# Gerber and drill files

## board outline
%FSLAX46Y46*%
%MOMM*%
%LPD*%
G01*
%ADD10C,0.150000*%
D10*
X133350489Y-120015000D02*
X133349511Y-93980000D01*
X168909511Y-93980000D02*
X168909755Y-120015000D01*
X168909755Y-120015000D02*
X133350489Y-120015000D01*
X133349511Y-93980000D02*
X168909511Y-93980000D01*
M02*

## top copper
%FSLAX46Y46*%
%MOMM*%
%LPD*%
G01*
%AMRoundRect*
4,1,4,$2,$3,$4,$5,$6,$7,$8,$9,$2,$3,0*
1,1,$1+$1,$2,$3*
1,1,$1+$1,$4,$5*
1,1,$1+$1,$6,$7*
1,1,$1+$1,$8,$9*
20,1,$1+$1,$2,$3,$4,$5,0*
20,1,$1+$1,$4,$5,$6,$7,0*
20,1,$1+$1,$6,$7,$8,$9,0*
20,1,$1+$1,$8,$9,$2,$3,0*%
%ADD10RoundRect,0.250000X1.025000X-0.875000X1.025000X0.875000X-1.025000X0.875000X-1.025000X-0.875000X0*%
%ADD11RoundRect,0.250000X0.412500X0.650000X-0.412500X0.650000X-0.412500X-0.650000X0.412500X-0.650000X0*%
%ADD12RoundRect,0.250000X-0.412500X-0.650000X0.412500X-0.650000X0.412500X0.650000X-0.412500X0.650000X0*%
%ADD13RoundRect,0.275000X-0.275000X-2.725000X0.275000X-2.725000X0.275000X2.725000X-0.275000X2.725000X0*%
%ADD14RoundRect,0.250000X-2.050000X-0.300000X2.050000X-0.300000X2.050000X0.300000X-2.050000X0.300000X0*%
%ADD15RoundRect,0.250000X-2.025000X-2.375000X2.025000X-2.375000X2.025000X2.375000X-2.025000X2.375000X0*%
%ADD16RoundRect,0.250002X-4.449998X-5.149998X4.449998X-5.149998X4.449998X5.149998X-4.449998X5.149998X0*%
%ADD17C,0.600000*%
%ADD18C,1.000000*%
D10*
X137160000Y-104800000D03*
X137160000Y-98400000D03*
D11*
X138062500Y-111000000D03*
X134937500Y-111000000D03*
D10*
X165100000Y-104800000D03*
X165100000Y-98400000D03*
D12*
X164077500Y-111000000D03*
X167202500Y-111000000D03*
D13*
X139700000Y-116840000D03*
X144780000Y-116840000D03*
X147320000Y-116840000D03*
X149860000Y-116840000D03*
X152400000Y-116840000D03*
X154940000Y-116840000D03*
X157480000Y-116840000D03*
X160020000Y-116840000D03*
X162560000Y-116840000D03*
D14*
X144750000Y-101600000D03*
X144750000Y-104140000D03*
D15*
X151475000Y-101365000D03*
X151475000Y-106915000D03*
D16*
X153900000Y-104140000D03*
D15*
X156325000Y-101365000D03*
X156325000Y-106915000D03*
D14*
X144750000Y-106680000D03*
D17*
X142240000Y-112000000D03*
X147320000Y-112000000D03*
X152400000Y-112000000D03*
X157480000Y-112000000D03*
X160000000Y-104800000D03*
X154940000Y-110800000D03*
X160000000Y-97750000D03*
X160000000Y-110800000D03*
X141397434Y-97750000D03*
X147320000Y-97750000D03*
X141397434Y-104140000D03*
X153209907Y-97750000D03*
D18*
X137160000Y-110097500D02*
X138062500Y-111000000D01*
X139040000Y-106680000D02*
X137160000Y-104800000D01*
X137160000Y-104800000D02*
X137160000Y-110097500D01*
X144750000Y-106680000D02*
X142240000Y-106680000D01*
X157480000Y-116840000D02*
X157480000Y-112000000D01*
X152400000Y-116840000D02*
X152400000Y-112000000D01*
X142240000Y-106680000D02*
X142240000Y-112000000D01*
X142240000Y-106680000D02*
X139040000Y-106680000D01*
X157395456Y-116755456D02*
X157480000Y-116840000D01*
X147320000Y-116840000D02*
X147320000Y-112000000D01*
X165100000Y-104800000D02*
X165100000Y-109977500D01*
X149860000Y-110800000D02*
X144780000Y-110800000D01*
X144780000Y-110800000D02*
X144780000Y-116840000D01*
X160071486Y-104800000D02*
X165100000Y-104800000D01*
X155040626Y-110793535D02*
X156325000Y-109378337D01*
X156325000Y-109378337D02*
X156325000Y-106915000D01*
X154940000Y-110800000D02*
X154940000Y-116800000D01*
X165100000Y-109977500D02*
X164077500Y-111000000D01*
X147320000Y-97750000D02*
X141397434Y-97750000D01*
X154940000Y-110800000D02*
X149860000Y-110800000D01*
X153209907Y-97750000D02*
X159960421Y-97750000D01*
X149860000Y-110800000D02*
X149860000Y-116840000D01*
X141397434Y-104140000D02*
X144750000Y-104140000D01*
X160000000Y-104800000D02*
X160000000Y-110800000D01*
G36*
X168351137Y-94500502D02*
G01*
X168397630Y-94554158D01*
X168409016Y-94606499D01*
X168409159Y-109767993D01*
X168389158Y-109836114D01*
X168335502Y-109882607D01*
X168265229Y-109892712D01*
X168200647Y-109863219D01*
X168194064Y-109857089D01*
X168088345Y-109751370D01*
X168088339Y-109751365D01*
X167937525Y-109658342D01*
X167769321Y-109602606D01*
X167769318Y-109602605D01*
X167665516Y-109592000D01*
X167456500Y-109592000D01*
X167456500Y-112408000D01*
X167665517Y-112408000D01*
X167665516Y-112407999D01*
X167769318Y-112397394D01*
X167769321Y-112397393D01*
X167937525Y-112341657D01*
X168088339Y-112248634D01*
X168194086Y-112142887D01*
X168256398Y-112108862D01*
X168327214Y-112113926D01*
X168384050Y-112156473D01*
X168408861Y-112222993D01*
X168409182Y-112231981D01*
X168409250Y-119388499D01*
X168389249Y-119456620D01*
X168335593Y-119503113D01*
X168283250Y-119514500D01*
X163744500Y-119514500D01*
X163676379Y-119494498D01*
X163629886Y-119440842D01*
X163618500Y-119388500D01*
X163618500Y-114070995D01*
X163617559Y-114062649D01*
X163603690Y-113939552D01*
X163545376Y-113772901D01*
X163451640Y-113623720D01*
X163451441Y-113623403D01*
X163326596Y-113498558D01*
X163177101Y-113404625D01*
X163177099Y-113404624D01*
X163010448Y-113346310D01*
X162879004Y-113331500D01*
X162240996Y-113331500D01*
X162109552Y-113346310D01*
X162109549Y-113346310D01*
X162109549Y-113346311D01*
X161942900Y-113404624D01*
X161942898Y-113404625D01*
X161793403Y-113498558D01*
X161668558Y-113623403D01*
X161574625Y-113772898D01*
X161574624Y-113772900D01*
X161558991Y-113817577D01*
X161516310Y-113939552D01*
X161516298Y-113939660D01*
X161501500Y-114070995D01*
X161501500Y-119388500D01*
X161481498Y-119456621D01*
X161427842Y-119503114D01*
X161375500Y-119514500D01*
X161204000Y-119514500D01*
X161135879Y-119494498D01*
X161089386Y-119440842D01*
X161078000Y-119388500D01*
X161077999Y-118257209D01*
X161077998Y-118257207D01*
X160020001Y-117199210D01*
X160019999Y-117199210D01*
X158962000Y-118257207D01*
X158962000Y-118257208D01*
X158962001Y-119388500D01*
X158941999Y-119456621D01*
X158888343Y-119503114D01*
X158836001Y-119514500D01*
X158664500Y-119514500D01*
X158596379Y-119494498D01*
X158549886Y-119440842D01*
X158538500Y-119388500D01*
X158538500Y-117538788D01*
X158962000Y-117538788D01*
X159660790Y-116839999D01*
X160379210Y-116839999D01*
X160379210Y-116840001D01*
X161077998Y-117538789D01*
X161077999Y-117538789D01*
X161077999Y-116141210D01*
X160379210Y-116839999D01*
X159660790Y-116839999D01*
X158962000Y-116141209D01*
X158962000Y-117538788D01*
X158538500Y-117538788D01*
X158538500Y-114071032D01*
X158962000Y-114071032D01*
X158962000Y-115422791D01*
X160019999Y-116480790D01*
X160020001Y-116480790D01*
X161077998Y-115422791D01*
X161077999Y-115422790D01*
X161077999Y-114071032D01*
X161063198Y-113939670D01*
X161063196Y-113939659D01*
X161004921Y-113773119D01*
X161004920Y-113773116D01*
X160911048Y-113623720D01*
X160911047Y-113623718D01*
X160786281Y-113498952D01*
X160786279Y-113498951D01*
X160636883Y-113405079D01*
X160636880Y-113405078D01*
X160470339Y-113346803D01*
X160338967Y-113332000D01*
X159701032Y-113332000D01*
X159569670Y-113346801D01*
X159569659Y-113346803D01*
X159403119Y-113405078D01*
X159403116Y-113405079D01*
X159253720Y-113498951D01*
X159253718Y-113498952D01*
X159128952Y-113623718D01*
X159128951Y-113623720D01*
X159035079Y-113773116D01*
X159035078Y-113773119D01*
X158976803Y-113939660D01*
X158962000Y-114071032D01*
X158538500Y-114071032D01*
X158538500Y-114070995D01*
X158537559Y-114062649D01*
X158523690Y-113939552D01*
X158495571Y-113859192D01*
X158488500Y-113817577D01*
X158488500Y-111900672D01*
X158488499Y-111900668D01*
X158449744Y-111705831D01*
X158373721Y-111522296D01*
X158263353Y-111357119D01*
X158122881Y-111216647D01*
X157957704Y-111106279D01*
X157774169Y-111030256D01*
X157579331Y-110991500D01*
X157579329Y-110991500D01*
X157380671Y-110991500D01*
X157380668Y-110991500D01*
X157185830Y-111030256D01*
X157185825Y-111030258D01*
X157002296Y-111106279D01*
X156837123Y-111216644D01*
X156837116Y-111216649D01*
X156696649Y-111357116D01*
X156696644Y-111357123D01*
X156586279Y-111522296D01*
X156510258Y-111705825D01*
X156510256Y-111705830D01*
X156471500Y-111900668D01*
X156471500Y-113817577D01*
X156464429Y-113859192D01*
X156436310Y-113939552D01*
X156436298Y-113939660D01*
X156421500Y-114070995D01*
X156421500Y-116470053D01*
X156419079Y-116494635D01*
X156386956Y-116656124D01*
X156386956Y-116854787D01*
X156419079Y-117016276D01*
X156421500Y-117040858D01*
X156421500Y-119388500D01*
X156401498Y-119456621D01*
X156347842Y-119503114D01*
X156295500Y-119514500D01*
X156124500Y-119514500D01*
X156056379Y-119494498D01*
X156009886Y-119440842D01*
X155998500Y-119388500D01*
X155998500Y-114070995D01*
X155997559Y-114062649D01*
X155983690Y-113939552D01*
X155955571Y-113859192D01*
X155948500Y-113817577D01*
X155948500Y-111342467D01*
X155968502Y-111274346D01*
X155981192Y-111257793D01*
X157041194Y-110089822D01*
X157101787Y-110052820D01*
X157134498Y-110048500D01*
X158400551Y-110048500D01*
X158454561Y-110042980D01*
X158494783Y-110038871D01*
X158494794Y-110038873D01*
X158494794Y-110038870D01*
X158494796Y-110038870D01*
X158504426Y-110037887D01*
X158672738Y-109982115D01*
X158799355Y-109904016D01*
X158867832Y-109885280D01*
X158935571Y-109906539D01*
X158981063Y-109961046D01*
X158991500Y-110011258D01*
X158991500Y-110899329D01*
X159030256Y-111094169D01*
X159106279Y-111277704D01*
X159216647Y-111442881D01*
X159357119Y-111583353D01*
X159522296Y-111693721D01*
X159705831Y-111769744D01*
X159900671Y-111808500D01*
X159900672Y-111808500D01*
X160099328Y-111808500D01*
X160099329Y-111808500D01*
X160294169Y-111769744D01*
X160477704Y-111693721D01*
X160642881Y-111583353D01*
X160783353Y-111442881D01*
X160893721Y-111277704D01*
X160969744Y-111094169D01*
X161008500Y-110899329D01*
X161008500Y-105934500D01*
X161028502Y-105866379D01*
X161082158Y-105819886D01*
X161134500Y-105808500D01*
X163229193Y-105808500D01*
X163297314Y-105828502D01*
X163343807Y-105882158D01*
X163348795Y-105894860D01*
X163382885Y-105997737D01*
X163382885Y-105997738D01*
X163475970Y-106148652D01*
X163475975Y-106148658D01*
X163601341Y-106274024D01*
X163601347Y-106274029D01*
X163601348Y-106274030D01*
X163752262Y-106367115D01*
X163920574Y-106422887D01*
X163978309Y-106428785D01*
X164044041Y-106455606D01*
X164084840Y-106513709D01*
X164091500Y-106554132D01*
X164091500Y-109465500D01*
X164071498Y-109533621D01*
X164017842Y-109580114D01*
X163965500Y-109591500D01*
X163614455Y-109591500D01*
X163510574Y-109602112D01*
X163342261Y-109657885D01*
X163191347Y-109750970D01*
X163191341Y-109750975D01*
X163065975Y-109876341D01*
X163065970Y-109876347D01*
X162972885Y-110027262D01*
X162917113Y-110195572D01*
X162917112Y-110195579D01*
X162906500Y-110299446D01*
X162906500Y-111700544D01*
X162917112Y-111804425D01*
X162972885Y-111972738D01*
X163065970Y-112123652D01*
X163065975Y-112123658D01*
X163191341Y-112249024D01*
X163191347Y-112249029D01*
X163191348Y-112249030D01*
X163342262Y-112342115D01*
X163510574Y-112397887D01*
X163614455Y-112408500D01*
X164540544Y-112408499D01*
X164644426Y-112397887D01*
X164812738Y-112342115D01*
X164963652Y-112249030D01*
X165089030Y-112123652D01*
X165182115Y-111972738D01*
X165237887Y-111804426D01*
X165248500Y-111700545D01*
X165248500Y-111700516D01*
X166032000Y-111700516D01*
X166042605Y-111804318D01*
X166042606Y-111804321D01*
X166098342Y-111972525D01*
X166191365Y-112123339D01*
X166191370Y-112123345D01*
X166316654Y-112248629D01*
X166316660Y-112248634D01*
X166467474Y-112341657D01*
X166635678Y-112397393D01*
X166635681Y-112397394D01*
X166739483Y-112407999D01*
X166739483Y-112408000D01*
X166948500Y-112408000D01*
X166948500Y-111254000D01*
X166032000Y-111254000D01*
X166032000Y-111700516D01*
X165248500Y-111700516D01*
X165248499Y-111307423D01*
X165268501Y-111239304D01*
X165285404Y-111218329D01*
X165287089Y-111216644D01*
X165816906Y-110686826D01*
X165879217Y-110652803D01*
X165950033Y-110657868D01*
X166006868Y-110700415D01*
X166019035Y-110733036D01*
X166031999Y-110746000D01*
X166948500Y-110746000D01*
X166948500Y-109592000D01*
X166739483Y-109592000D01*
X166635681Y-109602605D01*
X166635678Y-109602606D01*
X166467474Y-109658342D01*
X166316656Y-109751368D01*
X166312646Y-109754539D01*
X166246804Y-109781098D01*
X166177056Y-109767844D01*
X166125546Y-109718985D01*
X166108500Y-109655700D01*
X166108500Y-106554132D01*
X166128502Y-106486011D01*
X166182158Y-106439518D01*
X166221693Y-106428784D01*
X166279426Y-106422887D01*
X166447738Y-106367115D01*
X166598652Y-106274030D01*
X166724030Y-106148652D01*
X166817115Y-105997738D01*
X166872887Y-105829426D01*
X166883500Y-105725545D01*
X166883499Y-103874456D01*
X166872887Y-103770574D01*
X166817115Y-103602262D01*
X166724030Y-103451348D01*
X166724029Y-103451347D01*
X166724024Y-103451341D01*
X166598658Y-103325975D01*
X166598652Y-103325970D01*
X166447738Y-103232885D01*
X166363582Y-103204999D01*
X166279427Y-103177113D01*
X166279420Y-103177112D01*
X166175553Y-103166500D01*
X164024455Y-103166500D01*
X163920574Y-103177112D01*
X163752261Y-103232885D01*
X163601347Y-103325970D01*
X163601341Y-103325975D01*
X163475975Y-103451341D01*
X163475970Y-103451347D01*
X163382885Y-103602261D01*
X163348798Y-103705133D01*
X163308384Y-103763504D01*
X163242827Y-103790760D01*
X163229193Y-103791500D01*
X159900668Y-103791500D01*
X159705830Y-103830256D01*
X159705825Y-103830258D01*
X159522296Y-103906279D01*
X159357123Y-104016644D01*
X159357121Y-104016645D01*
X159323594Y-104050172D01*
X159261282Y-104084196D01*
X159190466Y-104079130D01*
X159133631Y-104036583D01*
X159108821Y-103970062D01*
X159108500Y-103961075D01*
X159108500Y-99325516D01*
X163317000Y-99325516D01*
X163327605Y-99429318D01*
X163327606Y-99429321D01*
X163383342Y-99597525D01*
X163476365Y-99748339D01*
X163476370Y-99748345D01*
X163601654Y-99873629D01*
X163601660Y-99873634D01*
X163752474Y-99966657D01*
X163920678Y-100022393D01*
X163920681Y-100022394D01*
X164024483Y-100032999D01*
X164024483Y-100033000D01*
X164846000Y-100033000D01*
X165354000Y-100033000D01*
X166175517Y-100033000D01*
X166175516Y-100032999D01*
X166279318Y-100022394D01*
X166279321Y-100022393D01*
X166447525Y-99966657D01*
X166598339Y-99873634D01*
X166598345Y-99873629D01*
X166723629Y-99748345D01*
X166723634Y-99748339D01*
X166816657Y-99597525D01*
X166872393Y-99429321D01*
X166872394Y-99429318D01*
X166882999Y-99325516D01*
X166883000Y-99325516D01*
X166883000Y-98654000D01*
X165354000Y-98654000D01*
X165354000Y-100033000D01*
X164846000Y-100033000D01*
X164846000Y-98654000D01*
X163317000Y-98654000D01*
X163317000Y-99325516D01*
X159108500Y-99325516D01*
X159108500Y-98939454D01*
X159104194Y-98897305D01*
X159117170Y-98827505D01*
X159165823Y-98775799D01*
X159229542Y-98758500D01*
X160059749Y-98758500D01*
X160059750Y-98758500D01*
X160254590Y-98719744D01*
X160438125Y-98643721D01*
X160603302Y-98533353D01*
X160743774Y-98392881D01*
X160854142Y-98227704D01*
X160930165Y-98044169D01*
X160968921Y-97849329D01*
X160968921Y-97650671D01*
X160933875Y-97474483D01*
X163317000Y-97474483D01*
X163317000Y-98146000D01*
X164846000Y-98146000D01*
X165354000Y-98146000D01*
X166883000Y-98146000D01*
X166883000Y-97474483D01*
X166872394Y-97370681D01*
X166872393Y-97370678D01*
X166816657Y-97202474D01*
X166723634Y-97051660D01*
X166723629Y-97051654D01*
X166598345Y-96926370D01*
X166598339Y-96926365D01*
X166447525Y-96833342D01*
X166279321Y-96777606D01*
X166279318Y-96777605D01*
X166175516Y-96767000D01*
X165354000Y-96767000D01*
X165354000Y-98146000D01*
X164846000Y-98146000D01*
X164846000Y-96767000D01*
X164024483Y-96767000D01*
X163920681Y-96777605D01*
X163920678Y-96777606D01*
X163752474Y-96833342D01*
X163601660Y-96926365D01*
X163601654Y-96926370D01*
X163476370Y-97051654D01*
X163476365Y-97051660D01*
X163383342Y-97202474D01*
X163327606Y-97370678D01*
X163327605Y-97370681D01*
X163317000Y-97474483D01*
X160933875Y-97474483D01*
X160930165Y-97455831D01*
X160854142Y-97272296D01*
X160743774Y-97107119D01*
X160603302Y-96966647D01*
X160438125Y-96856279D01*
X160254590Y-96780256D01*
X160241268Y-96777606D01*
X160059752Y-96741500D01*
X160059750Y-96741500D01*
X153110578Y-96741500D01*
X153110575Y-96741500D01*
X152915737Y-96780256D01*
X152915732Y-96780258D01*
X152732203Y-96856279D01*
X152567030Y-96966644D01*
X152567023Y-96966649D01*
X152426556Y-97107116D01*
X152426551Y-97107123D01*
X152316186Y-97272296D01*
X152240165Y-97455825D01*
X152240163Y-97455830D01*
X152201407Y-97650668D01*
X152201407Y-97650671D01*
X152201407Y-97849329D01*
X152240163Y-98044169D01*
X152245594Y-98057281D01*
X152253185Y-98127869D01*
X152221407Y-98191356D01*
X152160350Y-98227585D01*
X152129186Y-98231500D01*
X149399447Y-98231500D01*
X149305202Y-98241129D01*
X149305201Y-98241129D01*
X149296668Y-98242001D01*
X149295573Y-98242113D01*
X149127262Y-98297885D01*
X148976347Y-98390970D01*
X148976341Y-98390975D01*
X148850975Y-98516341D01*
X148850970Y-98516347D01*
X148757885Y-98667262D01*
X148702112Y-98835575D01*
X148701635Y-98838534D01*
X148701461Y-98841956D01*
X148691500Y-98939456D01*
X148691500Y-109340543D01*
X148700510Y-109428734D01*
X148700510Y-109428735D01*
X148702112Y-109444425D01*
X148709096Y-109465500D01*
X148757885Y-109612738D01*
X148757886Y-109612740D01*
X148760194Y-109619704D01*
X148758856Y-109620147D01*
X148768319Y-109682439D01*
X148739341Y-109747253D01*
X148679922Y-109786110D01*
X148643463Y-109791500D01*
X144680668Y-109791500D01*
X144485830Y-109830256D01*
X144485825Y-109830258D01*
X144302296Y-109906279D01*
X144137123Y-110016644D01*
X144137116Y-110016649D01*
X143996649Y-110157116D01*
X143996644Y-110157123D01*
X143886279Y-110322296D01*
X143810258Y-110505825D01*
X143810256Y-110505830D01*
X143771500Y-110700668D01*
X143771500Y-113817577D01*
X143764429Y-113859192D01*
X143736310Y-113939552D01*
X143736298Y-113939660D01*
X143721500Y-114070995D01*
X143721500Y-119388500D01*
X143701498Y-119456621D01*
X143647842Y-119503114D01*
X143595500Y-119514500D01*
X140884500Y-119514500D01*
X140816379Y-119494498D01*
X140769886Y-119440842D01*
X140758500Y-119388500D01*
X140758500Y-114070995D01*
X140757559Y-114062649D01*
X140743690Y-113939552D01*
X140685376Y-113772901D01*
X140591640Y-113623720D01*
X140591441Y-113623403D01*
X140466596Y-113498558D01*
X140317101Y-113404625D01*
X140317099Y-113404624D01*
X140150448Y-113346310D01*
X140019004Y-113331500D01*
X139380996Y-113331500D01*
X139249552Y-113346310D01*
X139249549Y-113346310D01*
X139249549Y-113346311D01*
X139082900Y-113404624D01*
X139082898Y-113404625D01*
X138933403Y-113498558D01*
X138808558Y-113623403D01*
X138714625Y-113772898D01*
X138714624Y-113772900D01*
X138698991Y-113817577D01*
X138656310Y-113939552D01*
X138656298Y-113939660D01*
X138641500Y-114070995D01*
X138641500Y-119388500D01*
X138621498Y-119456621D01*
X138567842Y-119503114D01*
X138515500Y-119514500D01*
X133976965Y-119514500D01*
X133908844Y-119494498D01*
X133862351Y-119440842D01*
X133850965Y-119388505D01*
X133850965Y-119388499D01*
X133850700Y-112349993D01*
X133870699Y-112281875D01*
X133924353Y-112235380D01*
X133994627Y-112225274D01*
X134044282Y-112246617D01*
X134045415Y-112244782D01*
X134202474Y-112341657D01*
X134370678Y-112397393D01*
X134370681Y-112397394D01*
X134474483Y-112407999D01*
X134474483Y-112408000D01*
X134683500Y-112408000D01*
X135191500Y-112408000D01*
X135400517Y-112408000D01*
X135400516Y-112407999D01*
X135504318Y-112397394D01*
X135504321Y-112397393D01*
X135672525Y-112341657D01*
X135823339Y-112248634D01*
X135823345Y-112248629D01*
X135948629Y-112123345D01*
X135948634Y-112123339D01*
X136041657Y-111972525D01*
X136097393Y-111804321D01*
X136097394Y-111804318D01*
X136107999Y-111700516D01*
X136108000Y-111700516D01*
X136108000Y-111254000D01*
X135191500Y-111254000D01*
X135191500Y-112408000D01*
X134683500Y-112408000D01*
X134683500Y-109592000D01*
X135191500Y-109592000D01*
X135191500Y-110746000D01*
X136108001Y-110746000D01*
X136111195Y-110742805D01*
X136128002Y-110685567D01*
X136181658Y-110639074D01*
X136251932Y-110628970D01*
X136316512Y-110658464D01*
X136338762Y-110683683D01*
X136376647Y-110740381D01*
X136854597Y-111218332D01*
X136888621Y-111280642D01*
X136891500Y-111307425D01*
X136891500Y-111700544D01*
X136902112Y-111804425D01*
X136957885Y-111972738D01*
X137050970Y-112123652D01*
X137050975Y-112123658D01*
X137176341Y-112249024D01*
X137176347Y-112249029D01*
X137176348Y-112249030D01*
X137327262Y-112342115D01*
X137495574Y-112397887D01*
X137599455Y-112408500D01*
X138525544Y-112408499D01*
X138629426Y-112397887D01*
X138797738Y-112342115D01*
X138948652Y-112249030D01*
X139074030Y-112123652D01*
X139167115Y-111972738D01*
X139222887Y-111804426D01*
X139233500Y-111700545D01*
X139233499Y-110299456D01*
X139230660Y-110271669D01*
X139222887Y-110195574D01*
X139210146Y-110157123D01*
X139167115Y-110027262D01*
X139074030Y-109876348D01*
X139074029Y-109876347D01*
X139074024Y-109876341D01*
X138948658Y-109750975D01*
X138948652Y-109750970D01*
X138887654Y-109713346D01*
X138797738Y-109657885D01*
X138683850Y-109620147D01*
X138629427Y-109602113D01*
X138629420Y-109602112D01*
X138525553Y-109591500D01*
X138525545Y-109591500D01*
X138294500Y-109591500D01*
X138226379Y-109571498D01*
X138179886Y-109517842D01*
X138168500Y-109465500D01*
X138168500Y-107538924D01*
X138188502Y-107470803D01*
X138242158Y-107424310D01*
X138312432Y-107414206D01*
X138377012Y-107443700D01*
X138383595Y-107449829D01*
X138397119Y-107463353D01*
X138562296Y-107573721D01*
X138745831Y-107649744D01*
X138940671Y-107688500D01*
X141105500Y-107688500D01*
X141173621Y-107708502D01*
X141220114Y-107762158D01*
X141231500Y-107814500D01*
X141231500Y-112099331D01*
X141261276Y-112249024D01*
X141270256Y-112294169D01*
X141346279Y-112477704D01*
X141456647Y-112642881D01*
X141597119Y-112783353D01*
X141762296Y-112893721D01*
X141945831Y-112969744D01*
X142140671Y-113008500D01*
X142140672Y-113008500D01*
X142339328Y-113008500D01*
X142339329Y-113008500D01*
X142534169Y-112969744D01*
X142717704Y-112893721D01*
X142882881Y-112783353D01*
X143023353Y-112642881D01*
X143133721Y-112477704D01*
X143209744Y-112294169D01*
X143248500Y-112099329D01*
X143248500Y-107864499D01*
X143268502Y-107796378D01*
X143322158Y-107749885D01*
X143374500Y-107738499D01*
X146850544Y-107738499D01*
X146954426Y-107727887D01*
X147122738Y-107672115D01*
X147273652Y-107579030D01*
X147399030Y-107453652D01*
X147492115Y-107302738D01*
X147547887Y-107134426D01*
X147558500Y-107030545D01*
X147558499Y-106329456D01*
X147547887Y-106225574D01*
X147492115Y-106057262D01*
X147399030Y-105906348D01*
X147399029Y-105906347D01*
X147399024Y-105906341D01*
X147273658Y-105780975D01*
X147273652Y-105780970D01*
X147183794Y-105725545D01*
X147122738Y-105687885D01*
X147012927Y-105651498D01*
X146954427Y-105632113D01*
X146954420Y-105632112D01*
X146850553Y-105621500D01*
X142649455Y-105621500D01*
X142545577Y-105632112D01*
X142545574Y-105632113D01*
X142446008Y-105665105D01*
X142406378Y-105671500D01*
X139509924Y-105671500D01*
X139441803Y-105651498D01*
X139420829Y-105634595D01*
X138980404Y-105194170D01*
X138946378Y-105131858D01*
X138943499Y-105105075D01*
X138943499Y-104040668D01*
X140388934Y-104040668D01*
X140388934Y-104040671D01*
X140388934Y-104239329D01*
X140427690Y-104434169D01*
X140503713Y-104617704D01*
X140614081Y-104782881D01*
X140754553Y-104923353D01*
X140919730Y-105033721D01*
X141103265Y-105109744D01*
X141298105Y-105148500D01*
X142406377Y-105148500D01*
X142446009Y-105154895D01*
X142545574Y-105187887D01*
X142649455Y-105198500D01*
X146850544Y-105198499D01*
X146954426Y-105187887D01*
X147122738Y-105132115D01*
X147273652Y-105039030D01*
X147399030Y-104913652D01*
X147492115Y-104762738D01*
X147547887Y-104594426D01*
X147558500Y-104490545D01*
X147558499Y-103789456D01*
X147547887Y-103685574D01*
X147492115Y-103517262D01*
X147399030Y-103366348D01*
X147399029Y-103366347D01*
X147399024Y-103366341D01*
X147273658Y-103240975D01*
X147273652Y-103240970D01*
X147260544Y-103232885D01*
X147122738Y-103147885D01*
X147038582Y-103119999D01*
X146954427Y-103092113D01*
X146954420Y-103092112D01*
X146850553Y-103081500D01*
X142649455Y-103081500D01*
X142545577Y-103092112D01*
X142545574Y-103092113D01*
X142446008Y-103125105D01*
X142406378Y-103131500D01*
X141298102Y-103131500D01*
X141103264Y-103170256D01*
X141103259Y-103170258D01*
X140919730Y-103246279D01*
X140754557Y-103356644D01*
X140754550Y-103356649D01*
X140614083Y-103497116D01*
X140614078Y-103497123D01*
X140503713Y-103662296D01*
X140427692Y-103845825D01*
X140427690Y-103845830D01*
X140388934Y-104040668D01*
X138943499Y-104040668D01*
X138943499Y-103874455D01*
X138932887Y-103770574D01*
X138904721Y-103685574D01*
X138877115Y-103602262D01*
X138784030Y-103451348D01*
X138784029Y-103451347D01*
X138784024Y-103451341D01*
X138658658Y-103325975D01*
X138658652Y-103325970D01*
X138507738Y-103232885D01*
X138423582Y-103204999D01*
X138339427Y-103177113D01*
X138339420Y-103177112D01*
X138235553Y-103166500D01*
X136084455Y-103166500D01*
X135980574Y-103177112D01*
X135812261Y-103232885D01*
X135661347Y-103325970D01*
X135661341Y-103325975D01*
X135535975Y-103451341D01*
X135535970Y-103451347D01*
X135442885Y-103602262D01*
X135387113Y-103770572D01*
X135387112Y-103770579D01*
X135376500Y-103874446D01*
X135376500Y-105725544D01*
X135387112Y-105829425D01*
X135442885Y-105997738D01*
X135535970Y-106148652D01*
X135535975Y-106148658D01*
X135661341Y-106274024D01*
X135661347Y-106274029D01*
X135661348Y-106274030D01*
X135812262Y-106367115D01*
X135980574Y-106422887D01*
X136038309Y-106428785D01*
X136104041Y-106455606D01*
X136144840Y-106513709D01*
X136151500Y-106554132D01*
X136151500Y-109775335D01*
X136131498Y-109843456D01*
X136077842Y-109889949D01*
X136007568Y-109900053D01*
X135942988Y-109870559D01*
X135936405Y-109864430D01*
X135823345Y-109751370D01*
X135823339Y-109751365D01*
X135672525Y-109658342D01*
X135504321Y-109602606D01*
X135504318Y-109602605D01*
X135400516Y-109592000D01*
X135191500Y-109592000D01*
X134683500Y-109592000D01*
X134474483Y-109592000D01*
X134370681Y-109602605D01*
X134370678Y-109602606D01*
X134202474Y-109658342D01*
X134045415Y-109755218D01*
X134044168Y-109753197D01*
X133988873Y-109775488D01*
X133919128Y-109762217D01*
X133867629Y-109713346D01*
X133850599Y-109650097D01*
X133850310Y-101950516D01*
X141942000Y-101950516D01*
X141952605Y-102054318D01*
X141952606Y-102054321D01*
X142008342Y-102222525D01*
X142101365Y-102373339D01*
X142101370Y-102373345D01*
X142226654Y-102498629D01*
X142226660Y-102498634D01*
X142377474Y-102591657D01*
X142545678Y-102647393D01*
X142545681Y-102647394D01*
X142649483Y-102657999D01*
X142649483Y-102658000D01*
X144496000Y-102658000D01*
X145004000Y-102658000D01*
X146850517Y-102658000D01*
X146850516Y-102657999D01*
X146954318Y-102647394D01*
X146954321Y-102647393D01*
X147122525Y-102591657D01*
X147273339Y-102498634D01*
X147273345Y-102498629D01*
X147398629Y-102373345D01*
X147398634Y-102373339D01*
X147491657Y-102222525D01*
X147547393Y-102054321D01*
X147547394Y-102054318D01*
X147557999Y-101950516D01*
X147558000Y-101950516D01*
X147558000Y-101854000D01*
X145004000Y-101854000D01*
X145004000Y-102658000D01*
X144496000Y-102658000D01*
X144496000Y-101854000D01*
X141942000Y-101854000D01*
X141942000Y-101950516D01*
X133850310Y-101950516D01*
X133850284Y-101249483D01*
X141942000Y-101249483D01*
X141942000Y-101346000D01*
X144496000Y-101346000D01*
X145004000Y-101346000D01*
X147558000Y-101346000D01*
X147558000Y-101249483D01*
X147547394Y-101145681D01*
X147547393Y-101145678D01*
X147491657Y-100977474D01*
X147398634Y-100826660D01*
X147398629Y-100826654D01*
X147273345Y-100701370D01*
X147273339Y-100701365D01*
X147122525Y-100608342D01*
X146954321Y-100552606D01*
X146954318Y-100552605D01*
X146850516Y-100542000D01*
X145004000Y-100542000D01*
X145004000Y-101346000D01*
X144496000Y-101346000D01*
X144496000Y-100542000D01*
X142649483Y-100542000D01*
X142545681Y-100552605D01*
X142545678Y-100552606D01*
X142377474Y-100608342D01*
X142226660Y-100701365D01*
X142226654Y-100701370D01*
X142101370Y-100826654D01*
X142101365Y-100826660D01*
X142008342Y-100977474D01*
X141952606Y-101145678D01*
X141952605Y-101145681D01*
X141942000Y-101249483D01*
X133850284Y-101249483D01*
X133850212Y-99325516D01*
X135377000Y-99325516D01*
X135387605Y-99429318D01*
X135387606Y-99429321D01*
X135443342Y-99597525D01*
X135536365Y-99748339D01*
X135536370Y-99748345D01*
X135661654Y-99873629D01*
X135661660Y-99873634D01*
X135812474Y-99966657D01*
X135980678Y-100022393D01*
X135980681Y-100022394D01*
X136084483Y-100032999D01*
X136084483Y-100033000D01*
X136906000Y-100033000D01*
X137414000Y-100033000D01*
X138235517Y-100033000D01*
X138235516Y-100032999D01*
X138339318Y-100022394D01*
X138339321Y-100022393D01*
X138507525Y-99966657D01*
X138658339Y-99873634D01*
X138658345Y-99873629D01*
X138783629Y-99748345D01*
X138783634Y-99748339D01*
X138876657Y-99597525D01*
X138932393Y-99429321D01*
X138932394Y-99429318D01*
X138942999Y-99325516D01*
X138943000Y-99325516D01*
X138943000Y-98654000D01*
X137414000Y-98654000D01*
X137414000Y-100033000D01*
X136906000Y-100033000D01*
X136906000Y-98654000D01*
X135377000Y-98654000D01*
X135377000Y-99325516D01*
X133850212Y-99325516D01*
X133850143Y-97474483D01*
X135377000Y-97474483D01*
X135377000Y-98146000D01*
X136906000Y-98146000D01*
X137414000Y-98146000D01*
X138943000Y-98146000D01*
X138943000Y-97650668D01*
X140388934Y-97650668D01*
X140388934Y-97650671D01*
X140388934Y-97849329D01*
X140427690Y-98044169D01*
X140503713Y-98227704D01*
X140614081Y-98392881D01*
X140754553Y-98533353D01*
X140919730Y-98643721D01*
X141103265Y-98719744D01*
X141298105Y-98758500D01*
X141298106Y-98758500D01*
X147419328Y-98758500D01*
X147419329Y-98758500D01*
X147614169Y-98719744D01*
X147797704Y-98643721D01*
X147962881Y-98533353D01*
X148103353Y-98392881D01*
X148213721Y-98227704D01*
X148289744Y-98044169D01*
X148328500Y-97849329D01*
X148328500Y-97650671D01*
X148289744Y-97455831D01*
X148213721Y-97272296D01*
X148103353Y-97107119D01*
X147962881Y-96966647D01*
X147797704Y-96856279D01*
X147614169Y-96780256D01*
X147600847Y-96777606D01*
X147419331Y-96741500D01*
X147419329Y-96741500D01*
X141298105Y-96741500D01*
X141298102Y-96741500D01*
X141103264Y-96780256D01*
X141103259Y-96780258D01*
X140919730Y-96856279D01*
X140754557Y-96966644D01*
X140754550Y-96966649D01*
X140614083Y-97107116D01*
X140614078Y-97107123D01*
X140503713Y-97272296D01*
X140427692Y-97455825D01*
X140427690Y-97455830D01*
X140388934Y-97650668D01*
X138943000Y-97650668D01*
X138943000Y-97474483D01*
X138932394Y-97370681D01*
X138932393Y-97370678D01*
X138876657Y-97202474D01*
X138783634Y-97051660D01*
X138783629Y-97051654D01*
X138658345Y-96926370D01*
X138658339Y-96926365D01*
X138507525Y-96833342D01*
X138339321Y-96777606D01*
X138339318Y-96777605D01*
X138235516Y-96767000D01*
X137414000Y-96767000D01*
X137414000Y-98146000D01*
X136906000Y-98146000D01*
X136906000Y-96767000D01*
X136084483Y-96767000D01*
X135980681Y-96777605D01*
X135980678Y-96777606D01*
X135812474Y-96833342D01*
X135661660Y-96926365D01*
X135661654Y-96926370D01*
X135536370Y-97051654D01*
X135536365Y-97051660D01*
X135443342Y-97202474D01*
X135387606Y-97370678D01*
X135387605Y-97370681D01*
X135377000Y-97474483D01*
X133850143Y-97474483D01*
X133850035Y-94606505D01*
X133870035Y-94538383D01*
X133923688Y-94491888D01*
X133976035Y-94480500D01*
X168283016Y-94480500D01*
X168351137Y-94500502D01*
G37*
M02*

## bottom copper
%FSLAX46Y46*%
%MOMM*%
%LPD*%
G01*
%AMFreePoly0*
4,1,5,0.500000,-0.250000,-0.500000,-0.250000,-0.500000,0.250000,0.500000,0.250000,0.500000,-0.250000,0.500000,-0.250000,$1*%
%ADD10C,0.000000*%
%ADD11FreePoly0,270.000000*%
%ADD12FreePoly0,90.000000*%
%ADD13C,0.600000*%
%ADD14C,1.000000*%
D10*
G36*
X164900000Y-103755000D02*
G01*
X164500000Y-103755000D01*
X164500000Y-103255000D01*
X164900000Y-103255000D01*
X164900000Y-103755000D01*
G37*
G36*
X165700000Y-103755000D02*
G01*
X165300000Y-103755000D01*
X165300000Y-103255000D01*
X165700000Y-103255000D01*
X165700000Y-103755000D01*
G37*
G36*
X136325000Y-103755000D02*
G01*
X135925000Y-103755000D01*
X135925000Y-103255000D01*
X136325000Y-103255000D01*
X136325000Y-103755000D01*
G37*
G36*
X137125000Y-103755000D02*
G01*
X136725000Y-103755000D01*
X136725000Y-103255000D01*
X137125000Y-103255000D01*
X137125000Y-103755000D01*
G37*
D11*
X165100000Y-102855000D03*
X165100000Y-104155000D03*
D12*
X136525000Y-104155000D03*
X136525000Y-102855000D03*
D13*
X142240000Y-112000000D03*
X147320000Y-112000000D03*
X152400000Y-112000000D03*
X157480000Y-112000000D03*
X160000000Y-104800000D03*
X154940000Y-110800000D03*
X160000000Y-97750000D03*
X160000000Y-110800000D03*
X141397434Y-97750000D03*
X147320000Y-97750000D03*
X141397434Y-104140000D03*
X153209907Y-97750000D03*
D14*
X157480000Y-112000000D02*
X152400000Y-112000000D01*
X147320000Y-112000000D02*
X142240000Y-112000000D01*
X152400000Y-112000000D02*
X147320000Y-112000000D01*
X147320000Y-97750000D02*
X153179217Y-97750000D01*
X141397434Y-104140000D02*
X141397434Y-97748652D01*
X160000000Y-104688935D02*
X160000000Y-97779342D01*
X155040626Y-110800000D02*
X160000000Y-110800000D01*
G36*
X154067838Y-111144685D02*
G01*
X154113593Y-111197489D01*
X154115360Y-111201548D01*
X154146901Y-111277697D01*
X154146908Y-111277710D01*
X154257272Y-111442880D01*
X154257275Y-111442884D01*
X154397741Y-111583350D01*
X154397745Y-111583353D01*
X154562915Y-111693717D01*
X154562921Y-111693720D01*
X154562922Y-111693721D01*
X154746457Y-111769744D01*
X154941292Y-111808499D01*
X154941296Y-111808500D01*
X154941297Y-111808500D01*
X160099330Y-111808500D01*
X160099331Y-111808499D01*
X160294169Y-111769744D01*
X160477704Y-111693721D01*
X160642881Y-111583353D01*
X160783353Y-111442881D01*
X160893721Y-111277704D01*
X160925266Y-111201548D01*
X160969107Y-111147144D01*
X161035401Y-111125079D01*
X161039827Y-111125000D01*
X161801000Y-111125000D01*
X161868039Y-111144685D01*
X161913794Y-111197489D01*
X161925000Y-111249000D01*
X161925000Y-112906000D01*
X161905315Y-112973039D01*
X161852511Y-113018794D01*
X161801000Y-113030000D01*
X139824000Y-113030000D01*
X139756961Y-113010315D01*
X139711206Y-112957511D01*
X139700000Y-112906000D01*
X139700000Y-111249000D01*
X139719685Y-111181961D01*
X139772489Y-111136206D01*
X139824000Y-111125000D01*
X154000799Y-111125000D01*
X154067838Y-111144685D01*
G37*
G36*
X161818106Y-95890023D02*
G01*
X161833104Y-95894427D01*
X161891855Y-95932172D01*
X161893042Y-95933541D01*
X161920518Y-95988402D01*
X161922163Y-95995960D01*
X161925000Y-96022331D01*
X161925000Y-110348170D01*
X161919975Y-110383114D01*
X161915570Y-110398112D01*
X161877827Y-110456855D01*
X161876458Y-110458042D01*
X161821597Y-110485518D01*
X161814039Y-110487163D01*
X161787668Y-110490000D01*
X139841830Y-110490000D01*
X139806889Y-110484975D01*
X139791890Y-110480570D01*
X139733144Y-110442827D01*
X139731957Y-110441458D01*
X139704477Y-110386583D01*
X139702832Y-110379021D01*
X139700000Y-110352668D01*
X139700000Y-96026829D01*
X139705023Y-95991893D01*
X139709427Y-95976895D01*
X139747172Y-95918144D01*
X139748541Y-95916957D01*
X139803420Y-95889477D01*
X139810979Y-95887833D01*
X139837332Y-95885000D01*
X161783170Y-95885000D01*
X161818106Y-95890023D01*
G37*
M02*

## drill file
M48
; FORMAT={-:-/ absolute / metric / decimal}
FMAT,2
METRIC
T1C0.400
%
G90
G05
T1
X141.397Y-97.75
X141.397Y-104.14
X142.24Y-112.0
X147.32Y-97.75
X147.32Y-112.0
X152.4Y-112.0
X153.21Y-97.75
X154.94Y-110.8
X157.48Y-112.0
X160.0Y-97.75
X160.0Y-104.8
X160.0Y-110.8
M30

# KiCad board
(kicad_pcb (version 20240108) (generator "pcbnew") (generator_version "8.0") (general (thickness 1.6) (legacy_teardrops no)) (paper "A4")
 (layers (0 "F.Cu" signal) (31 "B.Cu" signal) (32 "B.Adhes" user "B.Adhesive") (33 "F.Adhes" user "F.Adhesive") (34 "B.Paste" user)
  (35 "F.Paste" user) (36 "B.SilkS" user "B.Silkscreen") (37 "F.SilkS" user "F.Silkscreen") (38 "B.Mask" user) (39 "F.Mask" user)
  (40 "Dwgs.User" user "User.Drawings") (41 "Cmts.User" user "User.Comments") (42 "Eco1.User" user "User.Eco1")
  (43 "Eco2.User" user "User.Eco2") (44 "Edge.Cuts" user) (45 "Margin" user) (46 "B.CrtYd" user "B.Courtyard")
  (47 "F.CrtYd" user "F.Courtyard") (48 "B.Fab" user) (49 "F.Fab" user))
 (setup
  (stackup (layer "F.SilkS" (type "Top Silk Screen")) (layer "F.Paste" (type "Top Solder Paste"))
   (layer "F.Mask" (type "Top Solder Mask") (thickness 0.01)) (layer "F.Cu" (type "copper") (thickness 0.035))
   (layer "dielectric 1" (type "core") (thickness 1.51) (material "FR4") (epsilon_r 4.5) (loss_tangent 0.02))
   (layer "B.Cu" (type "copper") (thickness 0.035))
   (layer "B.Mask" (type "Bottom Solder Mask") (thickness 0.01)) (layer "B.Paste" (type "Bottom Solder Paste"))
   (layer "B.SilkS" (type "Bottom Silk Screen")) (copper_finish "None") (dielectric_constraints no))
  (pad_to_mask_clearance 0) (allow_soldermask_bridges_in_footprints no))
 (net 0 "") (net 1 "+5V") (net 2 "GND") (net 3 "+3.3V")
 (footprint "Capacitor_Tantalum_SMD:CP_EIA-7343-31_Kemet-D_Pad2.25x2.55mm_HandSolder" (layer "F.Cu") (at 137.16 101.6 90)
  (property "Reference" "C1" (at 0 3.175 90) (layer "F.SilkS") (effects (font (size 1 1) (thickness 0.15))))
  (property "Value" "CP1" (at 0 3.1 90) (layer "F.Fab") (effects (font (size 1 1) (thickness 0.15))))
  (pad "1" smd roundrect (at -3.2 0 90) (size 2.25 2.55) (layers "F.Cu" "F.Paste" "F.Mask") (roundrect_rratio 0.111111) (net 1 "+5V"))
  (pad "2" smd roundrect (at 3.2 0 90) (size 2.25 2.55) (layers "F.Cu" "F.Paste" "F.Mask") (roundrect_rratio 0.111111) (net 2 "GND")))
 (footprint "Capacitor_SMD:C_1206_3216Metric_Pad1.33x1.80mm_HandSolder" (layer "F.Cu") (at 136.5 111 180)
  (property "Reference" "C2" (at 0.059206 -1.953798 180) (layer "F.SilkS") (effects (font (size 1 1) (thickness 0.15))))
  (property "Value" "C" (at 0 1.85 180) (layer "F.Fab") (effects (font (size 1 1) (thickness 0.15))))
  (pad "1" smd roundrect (at -1.5625 0 180) (size 1.325 1.8) (layers "F.Cu" "F.Paste" "F.Mask") (roundrect_rratio 0.188679) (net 1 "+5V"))
  (pad "2" smd roundrect (at 1.5625 0 180) (size 1.325 1.8) (layers "F.Cu" "F.Paste" "F.Mask") (roundrect_rratio 0.188679) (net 2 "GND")))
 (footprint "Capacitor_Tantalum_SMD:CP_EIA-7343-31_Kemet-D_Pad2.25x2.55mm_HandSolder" (layer "F.Cu") (at 165.1 101.6 90)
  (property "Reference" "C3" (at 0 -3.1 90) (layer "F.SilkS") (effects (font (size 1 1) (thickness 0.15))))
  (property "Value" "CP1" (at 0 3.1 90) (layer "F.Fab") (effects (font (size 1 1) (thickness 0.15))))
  (pad "1" smd roundrect (at -3.2 0 90) (size 2.25 2.55) (layers "F.Cu" "F.Paste" "F.Mask") (roundrect_rratio 0.111111) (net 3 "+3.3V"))
  (pad "2" smd roundrect (at 3.2 0 90) (size 2.25 2.55) (layers "F.Cu" "F.Paste" "F.Mask") (roundrect_rratio 0.111111) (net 2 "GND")))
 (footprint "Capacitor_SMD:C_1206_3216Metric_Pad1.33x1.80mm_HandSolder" (layer "F.Cu") (at 165.64 111)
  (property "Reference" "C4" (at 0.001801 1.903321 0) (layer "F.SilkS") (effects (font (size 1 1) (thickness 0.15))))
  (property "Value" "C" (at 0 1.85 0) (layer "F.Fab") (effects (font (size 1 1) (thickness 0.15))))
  (pad "1" smd roundrect (at -1.5625 0) (size 1.325 1.8) (layers "F.Cu" "F.Paste" "F.Mask") (roundrect_rratio 0.188679) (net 3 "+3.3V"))
  (pad "2" smd roundrect (at 1.5625 0) (size 1.325 1.8) (layers "F.Cu" "F.Paste" "F.Mask") (roundrect_rratio 0.188679) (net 2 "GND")))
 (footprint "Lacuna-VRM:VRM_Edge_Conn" (layer "F.Cu") (at 157.48 124.46)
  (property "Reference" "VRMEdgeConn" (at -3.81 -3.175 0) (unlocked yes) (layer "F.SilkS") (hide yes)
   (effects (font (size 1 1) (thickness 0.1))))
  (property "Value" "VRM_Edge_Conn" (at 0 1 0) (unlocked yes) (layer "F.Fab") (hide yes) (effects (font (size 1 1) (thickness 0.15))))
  (pad "VC1" smd roundrect (at -17.78 -7.62) (size 1.1 6) (layers "F.Cu" "F.Paste" "F.Mask") (roundrect_rratio 0.25)
   (thermal_bridge_angle 45))
  (pad "VC2" smd roundrect (at -12.7 -7.62) (size 1.1 6) (layers "F.Cu" "F.Paste" "F.Mask") (roundrect_rratio 0.25) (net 3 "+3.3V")
   (thermal_bridge_angle 45))
  (pad "VC3" smd roundrect (at -10.16 -7.62) (size 1.1 6) (layers "F.Cu" "F.Paste" "F.Mask") (roundrect_rratio 0.25) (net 1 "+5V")
   (thermal_bridge_angle 45))
  (pad "VC4" smd roundrect (at -7.62 -7.62) (size 1.1 6) (layers "F.Cu" "F.Paste" "F.Mask") (roundrect_rratio 0.25) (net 3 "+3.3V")
   (thermal_bridge_angle 45))
  (pad "VC5" smd roundrect (at -5.08 -7.62) (size 1.1 6) (layers "F.Cu" "F.Paste" "F.Mask") (roundrect_rratio 0.25) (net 1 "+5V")
   (thermal_bridge_angle 45))
  (pad "VC6" smd roundrect (at -2.54 -7.62) (size 1.1 6) (layers "F.Cu" "F.Paste" "F.Mask") (roundrect_rratio 0.25) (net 3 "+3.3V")
   (thermal_bridge_angle 45))
  (pad "VC7" smd roundrect (at 0 -7.62) (size 1.1 6) (layers "F.Cu" "F.Paste" "F.Mask") (roundrect_rratio 0.25) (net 1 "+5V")
   (thermal_bridge_angle 45))
  (pad "VC8" smd roundrect (at 2.54 -7.62) (size 1.1 6) (layers "F.Cu" "F.Paste" "F.Mask") (roundrect_rratio 0.25) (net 2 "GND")
   (thermal_bridge_angle 45))
  (pad "VC9" smd roundrect (at 5.08 -7.62) (size 1.1 6) (layers "F.Cu" "F.Paste" "F.Mask") (roundrect_rratio 0.25) (thermal_bridge_angle 45)))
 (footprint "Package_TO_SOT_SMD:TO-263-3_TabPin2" (layer "F.Cu") (at 152.4 104.14)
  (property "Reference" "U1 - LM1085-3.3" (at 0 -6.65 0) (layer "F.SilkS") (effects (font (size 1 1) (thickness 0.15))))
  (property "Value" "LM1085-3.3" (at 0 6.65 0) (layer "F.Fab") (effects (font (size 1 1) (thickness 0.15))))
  (pad "1" smd roundrect (at -7.65 -2.54) (size 4.6 1.1) (layers "F.Cu" "F.Paste" "F.Mask") (roundrect_rratio 0.227273) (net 2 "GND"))
  (pad "2" smd roundrect (at -7.65 0) (size 4.6 1.1) (layers "F.Cu" "F.Paste" "F.Mask") (roundrect_rratio 0.227273) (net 3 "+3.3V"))
  (pad "2" smd roundrect (at -0.925 -2.775) (size 4.55 5.25) (layers "F.Cu" "F.Paste") (roundrect_rratio 0.054945) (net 3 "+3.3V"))
  (pad "2" smd roundrect (at -0.925 2.775) (size 4.55 5.25) (layers "F.Cu" "F.Paste") (roundrect_rratio 0.054945) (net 3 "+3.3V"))
  (pad "2" smd roundrect (at 1.5 0) (size 9.4 10.8) (layers "F.Cu" "F.Mask") (roundrect_rratio 0.026596) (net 3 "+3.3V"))
  (pad "2" smd roundrect (at 3.925 -2.775) (size 4.55 5.25) (layers "F.Cu" "F.Paste") (roundrect_rratio 0.054945) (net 3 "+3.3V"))
  (pad "2" smd roundrect (at 3.925 2.775) (size 4.55 5.25) (layers "F.Cu" "F.Paste") (roundrect_rratio 0.054945) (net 3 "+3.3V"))
  (pad "3" smd roundrect (at -7.65 2.54) (size 4.6 1.1) (layers "F.Cu" "F.Paste" "F.Mask") (roundrect_rratio 0.227273) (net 1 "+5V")))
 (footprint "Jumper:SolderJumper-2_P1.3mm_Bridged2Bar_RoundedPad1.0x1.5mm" (layer "B.Cu") (at 165.1 103.505 -90)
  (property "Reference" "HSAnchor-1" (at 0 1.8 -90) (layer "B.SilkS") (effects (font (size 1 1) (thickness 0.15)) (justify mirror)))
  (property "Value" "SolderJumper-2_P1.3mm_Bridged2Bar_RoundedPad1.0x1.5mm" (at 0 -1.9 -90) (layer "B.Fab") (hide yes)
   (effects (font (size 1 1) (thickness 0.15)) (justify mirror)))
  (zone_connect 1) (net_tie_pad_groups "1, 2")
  (fp_poly (pts (xy -0.25 0.6) (xy 0.25 0.6) (xy 0.25 0.2) (xy -0.25 0.2)) (stroke (width 0) (type solid)) (fill solid) (layer "B.Cu"))
  (fp_poly (pts (xy -0.25 -0.2) (xy 0.25 -0.2) (xy 0.25 -0.6) (xy -0.25 -0.6)) (stroke (width 0) (type solid)) (fill solid) (layer "B.Cu"))
  (pad "1" smd custom (at -0.65 0 270) (size 1 0.5) (layers "B.Cu" "B.Mask") (zone_connect 2) (thermal_bridge_angle 45)
   (options (clearance outline) (anchor rect)) (primitives))
  (pad "2" smd custom (at 0.65 0 270) (size 1 0.5) (layers "B.Cu" "B.Mask") (zone_connect 2) (thermal_bridge_angle 45)
   (options (clearance outline) (anchor rect)) (primitives)))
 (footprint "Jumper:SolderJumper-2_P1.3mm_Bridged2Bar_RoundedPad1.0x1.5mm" (layer "B.Cu") (at 136.525 103.505 90)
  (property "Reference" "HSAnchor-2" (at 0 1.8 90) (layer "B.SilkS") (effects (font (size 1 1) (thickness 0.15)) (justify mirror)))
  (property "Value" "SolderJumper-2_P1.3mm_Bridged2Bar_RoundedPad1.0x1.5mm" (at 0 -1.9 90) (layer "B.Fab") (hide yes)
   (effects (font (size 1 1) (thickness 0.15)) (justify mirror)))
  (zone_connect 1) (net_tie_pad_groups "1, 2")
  (fp_poly (pts (xy -0.25 -0.2) (xy 0.25 -0.2) (xy 0.25 -0.6) (xy -0.25 -0.6)) (stroke (width 0) (type solid)) (fill solid) (layer "B.Cu"))
  (fp_poly (pts (xy -0.25 0.6) (xy 0.25 0.6) (xy 0.25 0.2) (xy -0.25 0.2)) (stroke (width 0) (type solid)) (fill solid) (layer "B.Cu"))
  (pad "1" smd custom (at -0.65 0 90) (size 1 0.5) (layers "B.Cu" "B.Mask") (zone_connect 2) (thermal_bridge_angle 45)
   (options (clearance outline) (anchor rect)) (primitives))
  (pad "2" smd custom (at 0.65 0 90) (size 1 0.5) (layers "B.Cu" "B.Mask") (zone_connect 2) (thermal_bridge_angle 45)
   (options (clearance outline) (anchor rect)) (primitives)))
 (gr_line (start 133.350489 120.015) (end 133.349511 93.98) (stroke (width 0.15) (type default)) (layer "Edge.Cuts"))
 (gr_line (start 168.909511 93.98) (end 168.909755 120.015) (stroke (width 0.15) (type default)) (layer "Edge.Cuts"))
 (gr_line (start 168.909755 120.015) (end 133.350489 120.015) (stroke (width 0.15) (type default)) (layer "Edge.Cuts"))
 (gr_line (start 133.349511 93.98) (end 168.909511 93.98) (stroke (width 0.15) (type default)) (layer "Edge.Cuts"))
 (segment (start 137.16 110.0975) (end 138.0625 111) (width 1) (layer "F.Cu") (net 1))
 (segment (start 139.04 106.68) (end 137.16 104.8) (width 1) (layer "F.Cu") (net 1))
 (segment (start 137.16 104.8) (end 137.16 110.0975) (width 1) (layer "F.Cu") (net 1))
 (segment (start 144.75 106.68) (end 142.24 106.68) (width 1) (layer "F.Cu") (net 1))
 (segment (start 157.48 116.84) (end 157.48 112) (width 1) (layer "F.Cu") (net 1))
 (segment (start 152.4 116.84) (end 152.4 112) (width 1) (layer "F.Cu") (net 1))
 (segment (start 142.24 106.68) (end 142.24 112) (width 1) (layer "F.Cu") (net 1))
 (segment (start 142.24 106.68) (end 139.04 106.68) (width 1) (layer "F.Cu") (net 1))
 (segment (start 157.395456 116.755456) (end 157.48 116.84) (width 1) (layer "F.Cu") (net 1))
 (segment (start 147.32 116.84) (end 147.32 112) (width 1) (layer "F.Cu") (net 1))
 (via (at 142.24 112) (size 0.6) (drill 0.4) (layers "F.Cu" "B.Cu") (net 1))
 (via (at 147.32 112) (size 0.6) (drill 0.4) (layers "F.Cu" "B.Cu") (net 1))
 (via (at 152.4 112) (size 0.6) (drill 0.4) (layers "F.Cu" "B.Cu") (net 1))
 (via (at 157.48 112) (size 0.6) (drill 0.4) (layers "F.Cu" "B.Cu") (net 1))
 (segment (start 157.48 112) (end 152.4 112) (width 1) (layer "B.Cu") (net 1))
 (segment (start 147.32 112) (end 142.24 112) (width 1) (layer "B.Cu") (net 1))
 (segment (start 152.4 112) (end 147.32 112) (width 1) (layer "B.Cu") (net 1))
 (segment (start 165.1 104.8) (end 165.1 109.9775) (width 1) (layer "F.Cu") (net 3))
 (segment (start 149.86 110.8) (end 144.78 110.8) (width 1) (layer "F.Cu") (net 3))
 (segment (start 144.78 110.8) (end 144.78 116.84) (width 1) (layer "F.Cu") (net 3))
 (segment (start 160.071486 104.8) (end 165.1 104.8) (width 1) (layer "F.Cu") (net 3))
 (segment (start 155.040626 110.793535) (end 156.325 109.378337) (width 1) (layer "F.Cu") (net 3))
 (segment (start 156.325 109.378337) (end 156.325 106.915) (width 1) (layer "F.Cu") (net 3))
 (segment (start 154.94 110.8) (end 154.94 116.8) (width 1) (layer "F.Cu") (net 3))
 (segment (start 165.1 109.9775) (end 164.0775 111) (width 1) (layer "F.Cu") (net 3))
 (segment (start 147.32 97.75) (end 141.397434 97.75) (width 1) (layer "F.Cu") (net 3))
 (segment (start 154.94 110.8) (end 149.86 110.8) (width 1) (layer "F.Cu") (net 3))
 (segment (start 153.209907 97.75) (end 159.960421 97.75) (width 1) (layer "F.Cu") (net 3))
 (segment (start 149.86 110.8) (end 149.86 116.84) (width 1) (layer "F.Cu") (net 3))
 (segment (start 141.397434 104.14) (end 144.75 104.14) (width 1) (layer "F.Cu") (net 3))
 (segment (start 160 104.8) (end 160 110.8) (width 1) (layer "F.Cu") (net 3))
 (via (at 160 104.8) (size 0.6) (drill 0.4) (layers "F.Cu" "B.Cu") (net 3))
 (via (at 154.94 110.8) (size 0.6) (drill 0.4) (layers "F.Cu" "B.Cu") (free yes) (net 3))
 (via (at 160 97.75) (size 0.6) (drill 0.4) (layers "F.Cu" "B.Cu") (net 3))
 (via (at 160 110.8) (size 0.6) (drill 0.4) (layers "F.Cu" "B.Cu") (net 3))
 (via (at 141.397434 97.75) (size 0.6) (drill 0.4) (layers "F.Cu" "B.Cu") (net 3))
 (via (at 147.32 97.75) (size 0.6) (drill 0.4) (layers "F.Cu" "B.Cu") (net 3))
 (via (at 141.397434 104.14) (size 0.6) (drill 0.4) (layers "F.Cu" "B.Cu") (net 3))
 (via (at 153.209907 97.75) (size 0.6) (drill 0.4) (layers "F.Cu" "B.Cu") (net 3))
 (segment (start 147.32 97.75) (end 153.179217 97.75) (width 1) (layer "B.Cu") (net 3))
 (segment (start 141.397434 104.14) (end 141.397434 97.748652) (width 1) (layer "B.Cu") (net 3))
 (segment (start 160 104.688935) (end 160 97.779342) (width 1) (layer "B.Cu") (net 3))
 (segment (start 155.040626 110.8) (end 160 110.8) (width 1) (layer "B.Cu") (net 3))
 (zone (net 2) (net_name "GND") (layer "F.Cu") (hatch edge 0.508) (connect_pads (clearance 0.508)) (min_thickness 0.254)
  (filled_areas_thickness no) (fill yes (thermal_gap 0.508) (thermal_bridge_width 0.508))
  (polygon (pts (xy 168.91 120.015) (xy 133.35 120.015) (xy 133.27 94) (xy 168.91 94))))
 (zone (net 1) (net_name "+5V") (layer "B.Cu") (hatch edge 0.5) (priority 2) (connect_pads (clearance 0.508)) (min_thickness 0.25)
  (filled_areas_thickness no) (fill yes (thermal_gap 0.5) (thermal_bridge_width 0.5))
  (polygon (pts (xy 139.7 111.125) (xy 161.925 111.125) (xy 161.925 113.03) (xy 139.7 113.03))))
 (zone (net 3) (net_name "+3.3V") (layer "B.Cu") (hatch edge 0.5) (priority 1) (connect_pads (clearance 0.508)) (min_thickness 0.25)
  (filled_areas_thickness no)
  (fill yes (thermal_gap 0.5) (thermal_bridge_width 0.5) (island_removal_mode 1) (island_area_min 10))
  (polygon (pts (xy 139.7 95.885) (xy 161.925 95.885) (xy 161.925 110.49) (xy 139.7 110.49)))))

